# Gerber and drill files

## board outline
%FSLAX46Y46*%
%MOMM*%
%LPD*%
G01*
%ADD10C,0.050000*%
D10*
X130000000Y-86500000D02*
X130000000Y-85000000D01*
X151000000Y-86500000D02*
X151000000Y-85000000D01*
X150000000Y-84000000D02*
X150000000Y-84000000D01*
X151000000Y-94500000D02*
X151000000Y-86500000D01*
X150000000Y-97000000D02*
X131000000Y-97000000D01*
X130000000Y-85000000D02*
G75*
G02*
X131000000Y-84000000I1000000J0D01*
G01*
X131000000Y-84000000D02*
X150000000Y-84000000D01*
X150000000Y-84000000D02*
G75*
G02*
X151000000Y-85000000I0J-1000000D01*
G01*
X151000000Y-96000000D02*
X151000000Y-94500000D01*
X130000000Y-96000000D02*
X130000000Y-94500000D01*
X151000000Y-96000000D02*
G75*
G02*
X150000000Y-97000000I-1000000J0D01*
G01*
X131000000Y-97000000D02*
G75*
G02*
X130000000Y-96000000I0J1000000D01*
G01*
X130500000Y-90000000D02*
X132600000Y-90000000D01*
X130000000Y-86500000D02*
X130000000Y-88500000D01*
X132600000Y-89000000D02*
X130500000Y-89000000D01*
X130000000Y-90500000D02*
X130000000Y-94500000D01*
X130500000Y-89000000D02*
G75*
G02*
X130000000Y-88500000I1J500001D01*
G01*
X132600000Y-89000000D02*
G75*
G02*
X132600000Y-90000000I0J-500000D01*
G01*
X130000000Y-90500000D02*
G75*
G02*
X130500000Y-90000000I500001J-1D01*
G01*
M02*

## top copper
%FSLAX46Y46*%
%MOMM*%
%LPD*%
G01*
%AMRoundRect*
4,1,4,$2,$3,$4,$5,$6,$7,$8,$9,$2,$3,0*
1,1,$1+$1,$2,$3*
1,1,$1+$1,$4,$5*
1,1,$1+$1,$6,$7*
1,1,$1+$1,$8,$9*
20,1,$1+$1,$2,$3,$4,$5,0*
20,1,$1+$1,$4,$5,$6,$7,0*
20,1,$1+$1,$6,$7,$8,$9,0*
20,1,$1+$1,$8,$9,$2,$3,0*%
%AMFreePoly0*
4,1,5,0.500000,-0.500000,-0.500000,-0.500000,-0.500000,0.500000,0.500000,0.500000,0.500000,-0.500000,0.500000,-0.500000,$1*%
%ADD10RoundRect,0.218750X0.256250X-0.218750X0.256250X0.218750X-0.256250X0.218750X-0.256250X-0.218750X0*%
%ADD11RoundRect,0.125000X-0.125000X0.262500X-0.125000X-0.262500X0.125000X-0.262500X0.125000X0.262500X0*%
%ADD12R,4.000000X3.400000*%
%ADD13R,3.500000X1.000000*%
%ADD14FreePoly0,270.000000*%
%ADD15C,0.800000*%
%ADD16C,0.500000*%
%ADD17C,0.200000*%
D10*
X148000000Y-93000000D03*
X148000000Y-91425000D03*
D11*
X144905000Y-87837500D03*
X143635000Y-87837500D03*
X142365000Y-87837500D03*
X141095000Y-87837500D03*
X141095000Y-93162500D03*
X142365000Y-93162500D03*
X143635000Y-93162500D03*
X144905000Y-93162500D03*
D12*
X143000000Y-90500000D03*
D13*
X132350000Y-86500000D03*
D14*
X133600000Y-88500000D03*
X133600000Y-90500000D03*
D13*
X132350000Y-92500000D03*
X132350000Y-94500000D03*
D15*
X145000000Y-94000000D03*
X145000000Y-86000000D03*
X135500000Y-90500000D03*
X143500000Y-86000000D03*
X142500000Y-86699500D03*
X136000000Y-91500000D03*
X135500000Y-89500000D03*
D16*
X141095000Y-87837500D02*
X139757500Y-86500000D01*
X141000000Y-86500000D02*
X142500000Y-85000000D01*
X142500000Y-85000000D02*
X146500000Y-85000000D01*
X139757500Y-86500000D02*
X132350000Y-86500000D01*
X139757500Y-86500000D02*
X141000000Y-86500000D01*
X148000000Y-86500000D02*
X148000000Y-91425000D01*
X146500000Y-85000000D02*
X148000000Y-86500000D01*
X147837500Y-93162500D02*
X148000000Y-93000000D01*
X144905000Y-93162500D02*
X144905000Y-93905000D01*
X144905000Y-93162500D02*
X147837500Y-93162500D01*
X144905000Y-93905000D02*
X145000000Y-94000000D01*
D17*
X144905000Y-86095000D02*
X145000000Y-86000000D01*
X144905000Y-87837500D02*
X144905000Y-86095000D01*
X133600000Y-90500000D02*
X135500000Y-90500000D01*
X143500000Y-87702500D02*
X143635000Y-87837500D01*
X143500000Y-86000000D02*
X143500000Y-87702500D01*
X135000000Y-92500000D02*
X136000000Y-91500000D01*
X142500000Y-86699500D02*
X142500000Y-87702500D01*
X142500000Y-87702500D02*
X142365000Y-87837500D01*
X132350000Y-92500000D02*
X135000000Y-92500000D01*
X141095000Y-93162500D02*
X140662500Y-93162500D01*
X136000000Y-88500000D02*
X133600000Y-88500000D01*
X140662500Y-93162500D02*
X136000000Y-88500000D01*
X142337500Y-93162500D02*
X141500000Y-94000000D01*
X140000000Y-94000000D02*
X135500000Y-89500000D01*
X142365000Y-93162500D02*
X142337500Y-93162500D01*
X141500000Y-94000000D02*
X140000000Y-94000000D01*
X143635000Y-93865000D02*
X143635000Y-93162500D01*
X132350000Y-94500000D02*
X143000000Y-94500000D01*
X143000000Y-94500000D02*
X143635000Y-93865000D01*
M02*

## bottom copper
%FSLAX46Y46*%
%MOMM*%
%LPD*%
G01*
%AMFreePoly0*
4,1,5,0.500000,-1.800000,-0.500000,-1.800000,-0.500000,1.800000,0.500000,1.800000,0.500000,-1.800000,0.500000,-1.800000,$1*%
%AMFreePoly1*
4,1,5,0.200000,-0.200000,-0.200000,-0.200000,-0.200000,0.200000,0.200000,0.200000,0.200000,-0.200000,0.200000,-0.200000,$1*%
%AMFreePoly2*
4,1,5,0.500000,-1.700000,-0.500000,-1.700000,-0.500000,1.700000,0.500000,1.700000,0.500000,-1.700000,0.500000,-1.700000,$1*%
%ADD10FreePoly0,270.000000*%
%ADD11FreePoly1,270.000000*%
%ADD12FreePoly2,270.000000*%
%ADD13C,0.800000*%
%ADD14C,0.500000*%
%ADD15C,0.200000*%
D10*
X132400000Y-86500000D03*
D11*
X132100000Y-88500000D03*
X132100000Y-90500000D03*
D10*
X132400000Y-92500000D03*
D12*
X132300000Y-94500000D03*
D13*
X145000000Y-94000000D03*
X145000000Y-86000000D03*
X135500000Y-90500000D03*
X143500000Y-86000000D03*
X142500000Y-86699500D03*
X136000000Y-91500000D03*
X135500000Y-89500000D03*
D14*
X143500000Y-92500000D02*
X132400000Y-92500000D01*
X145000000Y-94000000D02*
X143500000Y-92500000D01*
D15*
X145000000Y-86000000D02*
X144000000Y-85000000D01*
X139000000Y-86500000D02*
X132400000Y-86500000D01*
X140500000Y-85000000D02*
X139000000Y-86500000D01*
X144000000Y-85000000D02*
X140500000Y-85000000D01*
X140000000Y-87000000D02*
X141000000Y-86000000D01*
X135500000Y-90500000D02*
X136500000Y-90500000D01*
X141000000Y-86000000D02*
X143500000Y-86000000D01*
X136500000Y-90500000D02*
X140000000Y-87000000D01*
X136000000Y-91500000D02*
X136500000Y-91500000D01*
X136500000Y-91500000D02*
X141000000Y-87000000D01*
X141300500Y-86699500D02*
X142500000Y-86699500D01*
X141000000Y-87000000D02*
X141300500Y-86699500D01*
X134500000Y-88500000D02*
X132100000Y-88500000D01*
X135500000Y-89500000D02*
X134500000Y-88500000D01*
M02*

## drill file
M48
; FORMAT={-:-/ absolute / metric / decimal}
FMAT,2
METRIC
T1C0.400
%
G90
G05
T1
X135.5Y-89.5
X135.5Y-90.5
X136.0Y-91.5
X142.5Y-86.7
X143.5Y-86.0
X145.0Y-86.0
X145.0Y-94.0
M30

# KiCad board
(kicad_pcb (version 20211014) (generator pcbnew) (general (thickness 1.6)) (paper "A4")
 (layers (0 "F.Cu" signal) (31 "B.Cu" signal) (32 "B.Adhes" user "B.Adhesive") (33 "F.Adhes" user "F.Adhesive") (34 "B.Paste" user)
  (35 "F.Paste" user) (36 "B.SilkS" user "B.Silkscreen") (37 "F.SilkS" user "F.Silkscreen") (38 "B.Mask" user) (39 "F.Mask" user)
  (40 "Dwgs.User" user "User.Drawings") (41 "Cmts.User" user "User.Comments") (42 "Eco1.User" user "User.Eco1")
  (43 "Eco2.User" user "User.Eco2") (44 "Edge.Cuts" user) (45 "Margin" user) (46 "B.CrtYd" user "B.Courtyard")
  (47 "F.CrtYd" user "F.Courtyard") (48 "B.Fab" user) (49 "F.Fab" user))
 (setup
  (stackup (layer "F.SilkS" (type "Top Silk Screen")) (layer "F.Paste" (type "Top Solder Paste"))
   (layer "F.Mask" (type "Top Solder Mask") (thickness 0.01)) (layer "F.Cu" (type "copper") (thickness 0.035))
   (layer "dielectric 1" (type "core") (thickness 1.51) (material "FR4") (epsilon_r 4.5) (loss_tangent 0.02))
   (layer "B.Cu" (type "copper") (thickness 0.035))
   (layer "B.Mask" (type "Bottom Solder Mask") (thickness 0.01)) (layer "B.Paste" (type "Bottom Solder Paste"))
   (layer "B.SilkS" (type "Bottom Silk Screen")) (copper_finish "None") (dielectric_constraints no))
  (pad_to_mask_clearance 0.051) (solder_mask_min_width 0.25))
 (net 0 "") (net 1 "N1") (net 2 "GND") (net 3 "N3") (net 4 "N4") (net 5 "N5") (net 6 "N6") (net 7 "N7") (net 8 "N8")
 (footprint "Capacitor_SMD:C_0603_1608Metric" (layer "F.Cu") (at 148 92.2125 90)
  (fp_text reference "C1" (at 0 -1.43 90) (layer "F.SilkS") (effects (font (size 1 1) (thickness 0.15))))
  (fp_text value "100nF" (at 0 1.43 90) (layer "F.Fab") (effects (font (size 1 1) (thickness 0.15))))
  (pad "1" smd roundrect locked (at -0.7875 0 90) (size 0.875 0.95) (layers "F.Cu" "F.Paste" "F.Mask") (roundrect_rratio 0.25) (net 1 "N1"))
  (pad "2" smd roundrect locked (at 0.7875 0 90) (size 0.875 0.95) (layers "F.Cu" "F.Paste" "F.Mask") (roundrect_rratio 0.25) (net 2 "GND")))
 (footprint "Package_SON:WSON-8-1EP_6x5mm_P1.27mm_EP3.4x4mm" (layer "F.Cu") (at 143 90.5 -90)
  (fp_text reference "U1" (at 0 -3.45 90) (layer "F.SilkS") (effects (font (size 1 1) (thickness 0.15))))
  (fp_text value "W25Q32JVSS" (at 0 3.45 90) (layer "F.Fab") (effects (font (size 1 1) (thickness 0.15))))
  (pad "" smd roundrect locked (at 0.85 -1 270) (size 1.37 1.61) (layers "F.Paste") (roundrect_rratio 0.182482))
  (pad "" smd roundrect locked (at -0.85 -1 270) (size 1.37 1.61) (layers "F.Paste") (roundrect_rratio 0.182482))
  (pad "" smd roundrect locked (at 0.85 1 270) (size 1.37 1.61) (layers "F.Paste") (roundrect_rratio 0.182482))
  (pad "" smd roundrect locked (at -0.85 1 270) (size 1.37 1.61) (layers "F.Paste") (roundrect_rratio 0.182482))
  (pad "1" smd roundrect locked (at -2.6625 -1.905 270) (size 0.775 0.5) (layers "F.Cu" "F.Paste" "F.Mask") (roundrect_rratio 0.25)
   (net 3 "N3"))
  (pad "2" smd roundrect locked (at -2.6625 -0.635 270) (size 0.775 0.5) (layers "F.Cu" "F.Paste" "F.Mask") (roundrect_rratio 0.25)
   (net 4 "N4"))
  (pad "3" smd roundrect locked (at -2.6625 0.635 270) (size 0.775 0.5) (layers "F.Cu" "F.Paste" "F.Mask") (roundrect_rratio 0.25)
   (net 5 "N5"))
  (pad "4" smd roundrect locked (at -2.6625 1.905 270) (size 0.775 0.5) (layers "F.Cu" "F.Paste" "F.Mask") (roundrect_rratio 0.25)
   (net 2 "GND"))
  (pad "5" smd roundrect locked (at 2.6625 1.905 270) (size 0.775 0.5) (layers "F.Cu" "F.Paste" "F.Mask") (roundrect_rratio 0.25)
   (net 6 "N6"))
  (pad "6" smd roundrect locked (at 2.6625 0.635 270) (size 0.775 0.5) (layers "F.Cu" "F.Paste" "F.Mask") (roundrect_rratio 0.25)
   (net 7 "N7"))
  (pad "7" smd roundrect locked (at 2.6625 -0.635 270) (size 0.775 0.5) (layers "F.Cu" "F.Paste" "F.Mask") (roundrect_rratio 0.25)
   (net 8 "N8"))
  (pad "8" smd roundrect locked (at 2.6625 -1.905 270) (size 0.775 0.5) (layers "F.Cu" "F.Paste" "F.Mask") (roundrect_rratio 0.25)
   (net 1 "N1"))
  (pad "9" smd rect locked (at 0 0 270) (size 3.4 4) (layers "F.Cu" "F.Mask")))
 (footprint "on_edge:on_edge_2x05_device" (layer "F.Cu") (at 130 90.5 -90)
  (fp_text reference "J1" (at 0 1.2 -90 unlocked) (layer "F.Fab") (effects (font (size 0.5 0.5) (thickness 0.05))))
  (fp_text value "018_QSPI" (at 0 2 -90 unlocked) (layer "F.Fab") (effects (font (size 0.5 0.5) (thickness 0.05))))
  (fp_line (start -0.5 -0.5) (end -0.5 -2.6) (layer "Edge.Cuts") (width 0.05))
  (fp_line (start -4 0) (end -2 0) (layer "Edge.Cuts") (width 0.05))
  (fp_line (start -1.5 -2.6) (end -1.5 -0.5) (layer "Edge.Cuts") (width 0.05))
  (fp_line (start 0 0) (end 4 0) (layer "Edge.Cuts") (width 0.05))
  (fp_arc (start -1.5 -0.5) (mid -1.646447 -0.146447) (end -2 0) (layer "Edge.Cuts") (width 0.05))
  (fp_arc (start -1.5 -2.6) (mid -1 -3.1) (end -0.5 -2.6) (layer "Edge.Cuts") (width 0.05))
  (fp_arc (start 0 0) (mid -0.353553 -0.146447) (end -0.5 -0.5) (layer "Edge.Cuts") (width 0.05))
  (pad "1" smd rect locked (at -4 -2.35 90) (size 1 3.5) (layers "F.Cu" "F.Mask") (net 2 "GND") (zone_connect 0))
  (pad "2" smd custom locked (at -2 -3.6 270) (size 1 1) (layers "F.Cu" "F.Mask") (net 6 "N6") (zone_connect 0)
   (options (clearance outline) (anchor rect)) (primitives))
  (pad "3" smd custom locked (at 0 -3.6 270) (size 1 1) (layers "F.Cu" "F.Mask") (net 4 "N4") (zone_connect 0)
   (options (clearance outline) (anchor rect)) (primitives))
  (pad "4" smd rect locked (at 2 -2.35 90) (size 1 3.5) (layers "F.Cu" "F.Mask") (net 5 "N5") (zone_connect 0))
  (pad "5" smd rect locked (at 4 -2.35 90) (size 1 3.5) (layers "F.Cu" "F.Mask") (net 8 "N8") (zone_connect 0))
  (pad "6" smd custom locked (at -4 -2.4 270) (size 1 3.6) (layers "B.Cu" "B.Mask") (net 3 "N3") (zone_connect 0)
   (options (clearance outline) (anchor rect)) (primitives))
  (pad "7" smd custom locked (at -2 -2.1 270) (size 0.4 0.4) (layers "B.Cu" "B.Mask") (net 7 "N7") (zone_connect 0)
   (options (clearance outline) (anchor rect)) (primitives))
  (pad "8" smd custom locked (at 0 -2.1 270) (size 0.4 0.4) (layers "B.Cu" "B.Mask") (zone_connect 0)
   (options (clearance outline) (anchor rect)) (primitives))
  (pad "9" smd custom locked (at 2 -2.4 270) (size 1 3.6) (layers "B.Cu" "B.Mask") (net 1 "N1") (zone_connect 0)
   (options (clearance outline) (anchor rect)) (primitives))
  (pad "10" smd custom locked (at 4 -2.3 270) (size 1 3.4) (layers "B.Cu" "B.Mask") (zone_connect 0)
   (options (clearance outline) (anchor rect)) (primitives)))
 (gr_line (start 130 86.5) (end 130 85) (layer "Edge.Cuts") (width 0.05))
 (gr_line (start 151 86.5) (end 151 85) (layer "Edge.Cuts") (width 0.05))
 (gr_line (start 150 84) (end 150 84) (layer "Edge.Cuts") (width 0.05))
 (gr_line (start 151 94.5) (end 151 86.5) (layer "Edge.Cuts") (width 0.05))
 (gr_line (start 150 97) (end 131 97) (layer "Edge.Cuts") (width 0.05))
 (gr_arc (start 130 85) (mid 130.292893 84.292893) (end 131 84) (layer "Edge.Cuts") (width 0.05))
 (gr_line (start 131 84) (end 150 84) (layer "Edge.Cuts") (width 0.05))
 (gr_arc (start 150 84) (mid 150.707107 84.292893) (end 151 85) (layer "Edge.Cuts") (width 0.05))
 (gr_line (start 151 96) (end 151 94.5) (layer "Edge.Cuts") (width 0.05))
 (gr_line (start 130 96) (end 130 94.5) (layer "Edge.Cuts") (width 0.05))
 (gr_arc (start 151 96) (mid 150.707107 96.707107) (end 150 97) (layer "Edge.Cuts") (width 0.05))
 (gr_arc (start 131 97) (mid 130.292893 96.707107) (end 130 96) (layer "Edge.Cuts") (width 0.05))
 (segment (start 141.095 87.8375) (end 139.7575 86.5) (width 0.5) (layer "F.Cu") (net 2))
 (segment (start 141 86.5) (end 142.5 85) (width 0.5) (layer "F.Cu") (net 2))
 (segment (start 142.5 85) (end 146.5 85) (width 0.5) (layer "F.Cu") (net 2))
 (segment (start 139.7575 86.5) (end 132.35 86.5) (width 0.5) (layer "F.Cu") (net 2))
 (segment (start 139.7575 86.5) (end 141 86.5) (width 0.5) (layer "F.Cu") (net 2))
 (segment (start 148 86.5) (end 148 91.425) (width 0.5) (layer "F.Cu") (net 2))
 (segment (start 146.5 85) (end 148 86.5) (width 0.5) (layer "F.Cu") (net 2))
 (segment (start 147.8375 93.1625) (end 148 93) (width 0.5) (layer "F.Cu") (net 1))
 (segment (start 144.905 93.1625) (end 144.905 93.905) (width 0.5) (layer "F.Cu") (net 1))
 (segment (start 144.905 93.1625) (end 147.8375 93.1625) (width 0.5) (layer "F.Cu") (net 1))
 (segment (start 144.905 93.905) (end 145 94) (width 0.5) (layer "F.Cu") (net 1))
 (via (at 145 94) (size 0.8) (drill 0.4) (layers "F.Cu" "B.Cu") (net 1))
 (segment (start 143.5 92.5) (end 132.4 92.5) (width 0.5) (layer "B.Cu") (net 1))
 (segment (start 145 94) (end 143.5 92.5) (width 0.5) (layer "B.Cu") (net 1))
 (segment (start 144.905 86.095) (end 145 86) (width 0.2) (layer "F.Cu") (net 3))
 (segment (start 144.905 87.8375) (end 144.905 86.095) (width 0.2) (layer "F.Cu") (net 3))
 (via (at 145 86) (size 0.8) (drill 0.4) (layers "F.Cu" "B.Cu") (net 3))
 (segment (start 145 86) (end 144 85) (width 0.2) (layer "B.Cu") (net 3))
 (segment (start 139 86.5) (end 132.4 86.5) (width 0.2) (layer "B.Cu") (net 3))
 (segment (start 140.5 85) (end 139 86.5) (width 0.2) (layer "B.Cu") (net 3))
 (segment (start 144 85) (end 140.5 85) (width 0.2) (layer "B.Cu") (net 3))
 (segment (start 133.6 90.5) (end 135.5 90.5) (width 0.2) (layer "F.Cu") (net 4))
 (segment (start 143.5 87.7025) (end 143.635 87.8375) (width 0.2) (layer "F.Cu") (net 4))
 (segment (start 143.5 86) (end 143.5 87.7025) (width 0.2) (layer "F.Cu") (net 4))
 (via (at 135.5 90.5) (size 0.8) (drill 0.4) (layers "F.Cu" "B.Cu") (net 4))
 (via (at 143.5 86) (size 0.8) (drill 0.4) (layers "F.Cu" "B.Cu") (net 4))
 (segment (start 140 87) (end 141 86) (width 0.2) (layer "B.Cu") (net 4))
 (segment (start 135.5 90.5) (end 136.5 90.5) (width 0.2) (layer "B.Cu") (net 4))
 (segment (start 141 86) (end 143.5 86) (width 0.2) (layer "B.Cu") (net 4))
 (segment (start 136.5 90.5) (end 140 87) (width 0.2) (layer "B.Cu") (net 4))
 (segment (start 135 92.5) (end 136 91.5) (width 0.2) (layer "F.Cu") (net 5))
 (segment (start 142.5 86.6995) (end 142.5 87.7025) (width 0.2) (layer "F.Cu") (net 5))
 (segment (start 142.5 87.7025) (end 142.365 87.8375) (width 0.2) (layer "F.Cu") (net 5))
 (segment (start 132.35 92.5) (end 135 92.5) (width 0.2) (layer "F.Cu") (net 5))
 (via (at 142.5 86.6995) (size 0.8) (drill 0.4) (layers "F.Cu" "B.Cu") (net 5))
 (via (at 136 91.5) (size 0.8) (drill 0.4) (layers "F.Cu" "B.Cu") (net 5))
 (segment (start 136 91.5) (end 136.5 91.5) (width 0.2) (layer "B.Cu") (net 5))
 (segment (start 136.5 91.5) (end 141 87) (width 0.2) (layer "B.Cu") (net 5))
 (segment (start 141.3005 86.6995) (end 142.5 86.6995) (width 0.2) (layer "B.Cu") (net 5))
 (segment (start 141 87) (end 141.3005 86.6995) (width 0.2) (layer "B.Cu") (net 5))
 (segment (start 141.095 93.1625) (end 140.6625 93.1625) (width 0.2) (layer "F.Cu") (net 6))
 (segment (start 136 88.5) (end 133.6 88.5) (width 0.2) (layer "F.Cu") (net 6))
 (segment (start 140.6625 93.1625) (end 136 88.5) (width 0.2) (layer "F.Cu") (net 6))
 (segment (start 142.3375 93.1625) (end 141.5 94) (width 0.2) (layer "F.Cu") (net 7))
 (segment (start 140 94) (end 135.5 89.5) (width 0.2) (layer "F.Cu") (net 7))
 (segment (start 142.365 93.1625) (end 142.3375 93.1625) (width 0.2) (layer "F.Cu") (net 7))
 (segment (start 141.5 94) (end 140 94) (width 0.2) (layer "F.Cu") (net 7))
 (via (at 135.5 89.5) (size 0.8) (drill 0.4) (layers "F.Cu" "B.Cu") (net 7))
 (segment (start 134.5 88.5) (end 132.1 88.5) (width 0.2) (layer "B.Cu") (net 7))
 (segment (start 135.5 89.5) (end 134.5 88.5) (width 0.2) (layer "B.Cu") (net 7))
 (segment (start 143.635 93.865) (end 143.635 93.1625) (width 0.2) (layer "F.Cu") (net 8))
 (segment (start 132.35 94.5) (end 143 94.5) (width 0.2) (layer "F.Cu") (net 8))
 (segment (start 143 94.5) (end 143.635 93.865) (width 0.2) (layer "F.Cu") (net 8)))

